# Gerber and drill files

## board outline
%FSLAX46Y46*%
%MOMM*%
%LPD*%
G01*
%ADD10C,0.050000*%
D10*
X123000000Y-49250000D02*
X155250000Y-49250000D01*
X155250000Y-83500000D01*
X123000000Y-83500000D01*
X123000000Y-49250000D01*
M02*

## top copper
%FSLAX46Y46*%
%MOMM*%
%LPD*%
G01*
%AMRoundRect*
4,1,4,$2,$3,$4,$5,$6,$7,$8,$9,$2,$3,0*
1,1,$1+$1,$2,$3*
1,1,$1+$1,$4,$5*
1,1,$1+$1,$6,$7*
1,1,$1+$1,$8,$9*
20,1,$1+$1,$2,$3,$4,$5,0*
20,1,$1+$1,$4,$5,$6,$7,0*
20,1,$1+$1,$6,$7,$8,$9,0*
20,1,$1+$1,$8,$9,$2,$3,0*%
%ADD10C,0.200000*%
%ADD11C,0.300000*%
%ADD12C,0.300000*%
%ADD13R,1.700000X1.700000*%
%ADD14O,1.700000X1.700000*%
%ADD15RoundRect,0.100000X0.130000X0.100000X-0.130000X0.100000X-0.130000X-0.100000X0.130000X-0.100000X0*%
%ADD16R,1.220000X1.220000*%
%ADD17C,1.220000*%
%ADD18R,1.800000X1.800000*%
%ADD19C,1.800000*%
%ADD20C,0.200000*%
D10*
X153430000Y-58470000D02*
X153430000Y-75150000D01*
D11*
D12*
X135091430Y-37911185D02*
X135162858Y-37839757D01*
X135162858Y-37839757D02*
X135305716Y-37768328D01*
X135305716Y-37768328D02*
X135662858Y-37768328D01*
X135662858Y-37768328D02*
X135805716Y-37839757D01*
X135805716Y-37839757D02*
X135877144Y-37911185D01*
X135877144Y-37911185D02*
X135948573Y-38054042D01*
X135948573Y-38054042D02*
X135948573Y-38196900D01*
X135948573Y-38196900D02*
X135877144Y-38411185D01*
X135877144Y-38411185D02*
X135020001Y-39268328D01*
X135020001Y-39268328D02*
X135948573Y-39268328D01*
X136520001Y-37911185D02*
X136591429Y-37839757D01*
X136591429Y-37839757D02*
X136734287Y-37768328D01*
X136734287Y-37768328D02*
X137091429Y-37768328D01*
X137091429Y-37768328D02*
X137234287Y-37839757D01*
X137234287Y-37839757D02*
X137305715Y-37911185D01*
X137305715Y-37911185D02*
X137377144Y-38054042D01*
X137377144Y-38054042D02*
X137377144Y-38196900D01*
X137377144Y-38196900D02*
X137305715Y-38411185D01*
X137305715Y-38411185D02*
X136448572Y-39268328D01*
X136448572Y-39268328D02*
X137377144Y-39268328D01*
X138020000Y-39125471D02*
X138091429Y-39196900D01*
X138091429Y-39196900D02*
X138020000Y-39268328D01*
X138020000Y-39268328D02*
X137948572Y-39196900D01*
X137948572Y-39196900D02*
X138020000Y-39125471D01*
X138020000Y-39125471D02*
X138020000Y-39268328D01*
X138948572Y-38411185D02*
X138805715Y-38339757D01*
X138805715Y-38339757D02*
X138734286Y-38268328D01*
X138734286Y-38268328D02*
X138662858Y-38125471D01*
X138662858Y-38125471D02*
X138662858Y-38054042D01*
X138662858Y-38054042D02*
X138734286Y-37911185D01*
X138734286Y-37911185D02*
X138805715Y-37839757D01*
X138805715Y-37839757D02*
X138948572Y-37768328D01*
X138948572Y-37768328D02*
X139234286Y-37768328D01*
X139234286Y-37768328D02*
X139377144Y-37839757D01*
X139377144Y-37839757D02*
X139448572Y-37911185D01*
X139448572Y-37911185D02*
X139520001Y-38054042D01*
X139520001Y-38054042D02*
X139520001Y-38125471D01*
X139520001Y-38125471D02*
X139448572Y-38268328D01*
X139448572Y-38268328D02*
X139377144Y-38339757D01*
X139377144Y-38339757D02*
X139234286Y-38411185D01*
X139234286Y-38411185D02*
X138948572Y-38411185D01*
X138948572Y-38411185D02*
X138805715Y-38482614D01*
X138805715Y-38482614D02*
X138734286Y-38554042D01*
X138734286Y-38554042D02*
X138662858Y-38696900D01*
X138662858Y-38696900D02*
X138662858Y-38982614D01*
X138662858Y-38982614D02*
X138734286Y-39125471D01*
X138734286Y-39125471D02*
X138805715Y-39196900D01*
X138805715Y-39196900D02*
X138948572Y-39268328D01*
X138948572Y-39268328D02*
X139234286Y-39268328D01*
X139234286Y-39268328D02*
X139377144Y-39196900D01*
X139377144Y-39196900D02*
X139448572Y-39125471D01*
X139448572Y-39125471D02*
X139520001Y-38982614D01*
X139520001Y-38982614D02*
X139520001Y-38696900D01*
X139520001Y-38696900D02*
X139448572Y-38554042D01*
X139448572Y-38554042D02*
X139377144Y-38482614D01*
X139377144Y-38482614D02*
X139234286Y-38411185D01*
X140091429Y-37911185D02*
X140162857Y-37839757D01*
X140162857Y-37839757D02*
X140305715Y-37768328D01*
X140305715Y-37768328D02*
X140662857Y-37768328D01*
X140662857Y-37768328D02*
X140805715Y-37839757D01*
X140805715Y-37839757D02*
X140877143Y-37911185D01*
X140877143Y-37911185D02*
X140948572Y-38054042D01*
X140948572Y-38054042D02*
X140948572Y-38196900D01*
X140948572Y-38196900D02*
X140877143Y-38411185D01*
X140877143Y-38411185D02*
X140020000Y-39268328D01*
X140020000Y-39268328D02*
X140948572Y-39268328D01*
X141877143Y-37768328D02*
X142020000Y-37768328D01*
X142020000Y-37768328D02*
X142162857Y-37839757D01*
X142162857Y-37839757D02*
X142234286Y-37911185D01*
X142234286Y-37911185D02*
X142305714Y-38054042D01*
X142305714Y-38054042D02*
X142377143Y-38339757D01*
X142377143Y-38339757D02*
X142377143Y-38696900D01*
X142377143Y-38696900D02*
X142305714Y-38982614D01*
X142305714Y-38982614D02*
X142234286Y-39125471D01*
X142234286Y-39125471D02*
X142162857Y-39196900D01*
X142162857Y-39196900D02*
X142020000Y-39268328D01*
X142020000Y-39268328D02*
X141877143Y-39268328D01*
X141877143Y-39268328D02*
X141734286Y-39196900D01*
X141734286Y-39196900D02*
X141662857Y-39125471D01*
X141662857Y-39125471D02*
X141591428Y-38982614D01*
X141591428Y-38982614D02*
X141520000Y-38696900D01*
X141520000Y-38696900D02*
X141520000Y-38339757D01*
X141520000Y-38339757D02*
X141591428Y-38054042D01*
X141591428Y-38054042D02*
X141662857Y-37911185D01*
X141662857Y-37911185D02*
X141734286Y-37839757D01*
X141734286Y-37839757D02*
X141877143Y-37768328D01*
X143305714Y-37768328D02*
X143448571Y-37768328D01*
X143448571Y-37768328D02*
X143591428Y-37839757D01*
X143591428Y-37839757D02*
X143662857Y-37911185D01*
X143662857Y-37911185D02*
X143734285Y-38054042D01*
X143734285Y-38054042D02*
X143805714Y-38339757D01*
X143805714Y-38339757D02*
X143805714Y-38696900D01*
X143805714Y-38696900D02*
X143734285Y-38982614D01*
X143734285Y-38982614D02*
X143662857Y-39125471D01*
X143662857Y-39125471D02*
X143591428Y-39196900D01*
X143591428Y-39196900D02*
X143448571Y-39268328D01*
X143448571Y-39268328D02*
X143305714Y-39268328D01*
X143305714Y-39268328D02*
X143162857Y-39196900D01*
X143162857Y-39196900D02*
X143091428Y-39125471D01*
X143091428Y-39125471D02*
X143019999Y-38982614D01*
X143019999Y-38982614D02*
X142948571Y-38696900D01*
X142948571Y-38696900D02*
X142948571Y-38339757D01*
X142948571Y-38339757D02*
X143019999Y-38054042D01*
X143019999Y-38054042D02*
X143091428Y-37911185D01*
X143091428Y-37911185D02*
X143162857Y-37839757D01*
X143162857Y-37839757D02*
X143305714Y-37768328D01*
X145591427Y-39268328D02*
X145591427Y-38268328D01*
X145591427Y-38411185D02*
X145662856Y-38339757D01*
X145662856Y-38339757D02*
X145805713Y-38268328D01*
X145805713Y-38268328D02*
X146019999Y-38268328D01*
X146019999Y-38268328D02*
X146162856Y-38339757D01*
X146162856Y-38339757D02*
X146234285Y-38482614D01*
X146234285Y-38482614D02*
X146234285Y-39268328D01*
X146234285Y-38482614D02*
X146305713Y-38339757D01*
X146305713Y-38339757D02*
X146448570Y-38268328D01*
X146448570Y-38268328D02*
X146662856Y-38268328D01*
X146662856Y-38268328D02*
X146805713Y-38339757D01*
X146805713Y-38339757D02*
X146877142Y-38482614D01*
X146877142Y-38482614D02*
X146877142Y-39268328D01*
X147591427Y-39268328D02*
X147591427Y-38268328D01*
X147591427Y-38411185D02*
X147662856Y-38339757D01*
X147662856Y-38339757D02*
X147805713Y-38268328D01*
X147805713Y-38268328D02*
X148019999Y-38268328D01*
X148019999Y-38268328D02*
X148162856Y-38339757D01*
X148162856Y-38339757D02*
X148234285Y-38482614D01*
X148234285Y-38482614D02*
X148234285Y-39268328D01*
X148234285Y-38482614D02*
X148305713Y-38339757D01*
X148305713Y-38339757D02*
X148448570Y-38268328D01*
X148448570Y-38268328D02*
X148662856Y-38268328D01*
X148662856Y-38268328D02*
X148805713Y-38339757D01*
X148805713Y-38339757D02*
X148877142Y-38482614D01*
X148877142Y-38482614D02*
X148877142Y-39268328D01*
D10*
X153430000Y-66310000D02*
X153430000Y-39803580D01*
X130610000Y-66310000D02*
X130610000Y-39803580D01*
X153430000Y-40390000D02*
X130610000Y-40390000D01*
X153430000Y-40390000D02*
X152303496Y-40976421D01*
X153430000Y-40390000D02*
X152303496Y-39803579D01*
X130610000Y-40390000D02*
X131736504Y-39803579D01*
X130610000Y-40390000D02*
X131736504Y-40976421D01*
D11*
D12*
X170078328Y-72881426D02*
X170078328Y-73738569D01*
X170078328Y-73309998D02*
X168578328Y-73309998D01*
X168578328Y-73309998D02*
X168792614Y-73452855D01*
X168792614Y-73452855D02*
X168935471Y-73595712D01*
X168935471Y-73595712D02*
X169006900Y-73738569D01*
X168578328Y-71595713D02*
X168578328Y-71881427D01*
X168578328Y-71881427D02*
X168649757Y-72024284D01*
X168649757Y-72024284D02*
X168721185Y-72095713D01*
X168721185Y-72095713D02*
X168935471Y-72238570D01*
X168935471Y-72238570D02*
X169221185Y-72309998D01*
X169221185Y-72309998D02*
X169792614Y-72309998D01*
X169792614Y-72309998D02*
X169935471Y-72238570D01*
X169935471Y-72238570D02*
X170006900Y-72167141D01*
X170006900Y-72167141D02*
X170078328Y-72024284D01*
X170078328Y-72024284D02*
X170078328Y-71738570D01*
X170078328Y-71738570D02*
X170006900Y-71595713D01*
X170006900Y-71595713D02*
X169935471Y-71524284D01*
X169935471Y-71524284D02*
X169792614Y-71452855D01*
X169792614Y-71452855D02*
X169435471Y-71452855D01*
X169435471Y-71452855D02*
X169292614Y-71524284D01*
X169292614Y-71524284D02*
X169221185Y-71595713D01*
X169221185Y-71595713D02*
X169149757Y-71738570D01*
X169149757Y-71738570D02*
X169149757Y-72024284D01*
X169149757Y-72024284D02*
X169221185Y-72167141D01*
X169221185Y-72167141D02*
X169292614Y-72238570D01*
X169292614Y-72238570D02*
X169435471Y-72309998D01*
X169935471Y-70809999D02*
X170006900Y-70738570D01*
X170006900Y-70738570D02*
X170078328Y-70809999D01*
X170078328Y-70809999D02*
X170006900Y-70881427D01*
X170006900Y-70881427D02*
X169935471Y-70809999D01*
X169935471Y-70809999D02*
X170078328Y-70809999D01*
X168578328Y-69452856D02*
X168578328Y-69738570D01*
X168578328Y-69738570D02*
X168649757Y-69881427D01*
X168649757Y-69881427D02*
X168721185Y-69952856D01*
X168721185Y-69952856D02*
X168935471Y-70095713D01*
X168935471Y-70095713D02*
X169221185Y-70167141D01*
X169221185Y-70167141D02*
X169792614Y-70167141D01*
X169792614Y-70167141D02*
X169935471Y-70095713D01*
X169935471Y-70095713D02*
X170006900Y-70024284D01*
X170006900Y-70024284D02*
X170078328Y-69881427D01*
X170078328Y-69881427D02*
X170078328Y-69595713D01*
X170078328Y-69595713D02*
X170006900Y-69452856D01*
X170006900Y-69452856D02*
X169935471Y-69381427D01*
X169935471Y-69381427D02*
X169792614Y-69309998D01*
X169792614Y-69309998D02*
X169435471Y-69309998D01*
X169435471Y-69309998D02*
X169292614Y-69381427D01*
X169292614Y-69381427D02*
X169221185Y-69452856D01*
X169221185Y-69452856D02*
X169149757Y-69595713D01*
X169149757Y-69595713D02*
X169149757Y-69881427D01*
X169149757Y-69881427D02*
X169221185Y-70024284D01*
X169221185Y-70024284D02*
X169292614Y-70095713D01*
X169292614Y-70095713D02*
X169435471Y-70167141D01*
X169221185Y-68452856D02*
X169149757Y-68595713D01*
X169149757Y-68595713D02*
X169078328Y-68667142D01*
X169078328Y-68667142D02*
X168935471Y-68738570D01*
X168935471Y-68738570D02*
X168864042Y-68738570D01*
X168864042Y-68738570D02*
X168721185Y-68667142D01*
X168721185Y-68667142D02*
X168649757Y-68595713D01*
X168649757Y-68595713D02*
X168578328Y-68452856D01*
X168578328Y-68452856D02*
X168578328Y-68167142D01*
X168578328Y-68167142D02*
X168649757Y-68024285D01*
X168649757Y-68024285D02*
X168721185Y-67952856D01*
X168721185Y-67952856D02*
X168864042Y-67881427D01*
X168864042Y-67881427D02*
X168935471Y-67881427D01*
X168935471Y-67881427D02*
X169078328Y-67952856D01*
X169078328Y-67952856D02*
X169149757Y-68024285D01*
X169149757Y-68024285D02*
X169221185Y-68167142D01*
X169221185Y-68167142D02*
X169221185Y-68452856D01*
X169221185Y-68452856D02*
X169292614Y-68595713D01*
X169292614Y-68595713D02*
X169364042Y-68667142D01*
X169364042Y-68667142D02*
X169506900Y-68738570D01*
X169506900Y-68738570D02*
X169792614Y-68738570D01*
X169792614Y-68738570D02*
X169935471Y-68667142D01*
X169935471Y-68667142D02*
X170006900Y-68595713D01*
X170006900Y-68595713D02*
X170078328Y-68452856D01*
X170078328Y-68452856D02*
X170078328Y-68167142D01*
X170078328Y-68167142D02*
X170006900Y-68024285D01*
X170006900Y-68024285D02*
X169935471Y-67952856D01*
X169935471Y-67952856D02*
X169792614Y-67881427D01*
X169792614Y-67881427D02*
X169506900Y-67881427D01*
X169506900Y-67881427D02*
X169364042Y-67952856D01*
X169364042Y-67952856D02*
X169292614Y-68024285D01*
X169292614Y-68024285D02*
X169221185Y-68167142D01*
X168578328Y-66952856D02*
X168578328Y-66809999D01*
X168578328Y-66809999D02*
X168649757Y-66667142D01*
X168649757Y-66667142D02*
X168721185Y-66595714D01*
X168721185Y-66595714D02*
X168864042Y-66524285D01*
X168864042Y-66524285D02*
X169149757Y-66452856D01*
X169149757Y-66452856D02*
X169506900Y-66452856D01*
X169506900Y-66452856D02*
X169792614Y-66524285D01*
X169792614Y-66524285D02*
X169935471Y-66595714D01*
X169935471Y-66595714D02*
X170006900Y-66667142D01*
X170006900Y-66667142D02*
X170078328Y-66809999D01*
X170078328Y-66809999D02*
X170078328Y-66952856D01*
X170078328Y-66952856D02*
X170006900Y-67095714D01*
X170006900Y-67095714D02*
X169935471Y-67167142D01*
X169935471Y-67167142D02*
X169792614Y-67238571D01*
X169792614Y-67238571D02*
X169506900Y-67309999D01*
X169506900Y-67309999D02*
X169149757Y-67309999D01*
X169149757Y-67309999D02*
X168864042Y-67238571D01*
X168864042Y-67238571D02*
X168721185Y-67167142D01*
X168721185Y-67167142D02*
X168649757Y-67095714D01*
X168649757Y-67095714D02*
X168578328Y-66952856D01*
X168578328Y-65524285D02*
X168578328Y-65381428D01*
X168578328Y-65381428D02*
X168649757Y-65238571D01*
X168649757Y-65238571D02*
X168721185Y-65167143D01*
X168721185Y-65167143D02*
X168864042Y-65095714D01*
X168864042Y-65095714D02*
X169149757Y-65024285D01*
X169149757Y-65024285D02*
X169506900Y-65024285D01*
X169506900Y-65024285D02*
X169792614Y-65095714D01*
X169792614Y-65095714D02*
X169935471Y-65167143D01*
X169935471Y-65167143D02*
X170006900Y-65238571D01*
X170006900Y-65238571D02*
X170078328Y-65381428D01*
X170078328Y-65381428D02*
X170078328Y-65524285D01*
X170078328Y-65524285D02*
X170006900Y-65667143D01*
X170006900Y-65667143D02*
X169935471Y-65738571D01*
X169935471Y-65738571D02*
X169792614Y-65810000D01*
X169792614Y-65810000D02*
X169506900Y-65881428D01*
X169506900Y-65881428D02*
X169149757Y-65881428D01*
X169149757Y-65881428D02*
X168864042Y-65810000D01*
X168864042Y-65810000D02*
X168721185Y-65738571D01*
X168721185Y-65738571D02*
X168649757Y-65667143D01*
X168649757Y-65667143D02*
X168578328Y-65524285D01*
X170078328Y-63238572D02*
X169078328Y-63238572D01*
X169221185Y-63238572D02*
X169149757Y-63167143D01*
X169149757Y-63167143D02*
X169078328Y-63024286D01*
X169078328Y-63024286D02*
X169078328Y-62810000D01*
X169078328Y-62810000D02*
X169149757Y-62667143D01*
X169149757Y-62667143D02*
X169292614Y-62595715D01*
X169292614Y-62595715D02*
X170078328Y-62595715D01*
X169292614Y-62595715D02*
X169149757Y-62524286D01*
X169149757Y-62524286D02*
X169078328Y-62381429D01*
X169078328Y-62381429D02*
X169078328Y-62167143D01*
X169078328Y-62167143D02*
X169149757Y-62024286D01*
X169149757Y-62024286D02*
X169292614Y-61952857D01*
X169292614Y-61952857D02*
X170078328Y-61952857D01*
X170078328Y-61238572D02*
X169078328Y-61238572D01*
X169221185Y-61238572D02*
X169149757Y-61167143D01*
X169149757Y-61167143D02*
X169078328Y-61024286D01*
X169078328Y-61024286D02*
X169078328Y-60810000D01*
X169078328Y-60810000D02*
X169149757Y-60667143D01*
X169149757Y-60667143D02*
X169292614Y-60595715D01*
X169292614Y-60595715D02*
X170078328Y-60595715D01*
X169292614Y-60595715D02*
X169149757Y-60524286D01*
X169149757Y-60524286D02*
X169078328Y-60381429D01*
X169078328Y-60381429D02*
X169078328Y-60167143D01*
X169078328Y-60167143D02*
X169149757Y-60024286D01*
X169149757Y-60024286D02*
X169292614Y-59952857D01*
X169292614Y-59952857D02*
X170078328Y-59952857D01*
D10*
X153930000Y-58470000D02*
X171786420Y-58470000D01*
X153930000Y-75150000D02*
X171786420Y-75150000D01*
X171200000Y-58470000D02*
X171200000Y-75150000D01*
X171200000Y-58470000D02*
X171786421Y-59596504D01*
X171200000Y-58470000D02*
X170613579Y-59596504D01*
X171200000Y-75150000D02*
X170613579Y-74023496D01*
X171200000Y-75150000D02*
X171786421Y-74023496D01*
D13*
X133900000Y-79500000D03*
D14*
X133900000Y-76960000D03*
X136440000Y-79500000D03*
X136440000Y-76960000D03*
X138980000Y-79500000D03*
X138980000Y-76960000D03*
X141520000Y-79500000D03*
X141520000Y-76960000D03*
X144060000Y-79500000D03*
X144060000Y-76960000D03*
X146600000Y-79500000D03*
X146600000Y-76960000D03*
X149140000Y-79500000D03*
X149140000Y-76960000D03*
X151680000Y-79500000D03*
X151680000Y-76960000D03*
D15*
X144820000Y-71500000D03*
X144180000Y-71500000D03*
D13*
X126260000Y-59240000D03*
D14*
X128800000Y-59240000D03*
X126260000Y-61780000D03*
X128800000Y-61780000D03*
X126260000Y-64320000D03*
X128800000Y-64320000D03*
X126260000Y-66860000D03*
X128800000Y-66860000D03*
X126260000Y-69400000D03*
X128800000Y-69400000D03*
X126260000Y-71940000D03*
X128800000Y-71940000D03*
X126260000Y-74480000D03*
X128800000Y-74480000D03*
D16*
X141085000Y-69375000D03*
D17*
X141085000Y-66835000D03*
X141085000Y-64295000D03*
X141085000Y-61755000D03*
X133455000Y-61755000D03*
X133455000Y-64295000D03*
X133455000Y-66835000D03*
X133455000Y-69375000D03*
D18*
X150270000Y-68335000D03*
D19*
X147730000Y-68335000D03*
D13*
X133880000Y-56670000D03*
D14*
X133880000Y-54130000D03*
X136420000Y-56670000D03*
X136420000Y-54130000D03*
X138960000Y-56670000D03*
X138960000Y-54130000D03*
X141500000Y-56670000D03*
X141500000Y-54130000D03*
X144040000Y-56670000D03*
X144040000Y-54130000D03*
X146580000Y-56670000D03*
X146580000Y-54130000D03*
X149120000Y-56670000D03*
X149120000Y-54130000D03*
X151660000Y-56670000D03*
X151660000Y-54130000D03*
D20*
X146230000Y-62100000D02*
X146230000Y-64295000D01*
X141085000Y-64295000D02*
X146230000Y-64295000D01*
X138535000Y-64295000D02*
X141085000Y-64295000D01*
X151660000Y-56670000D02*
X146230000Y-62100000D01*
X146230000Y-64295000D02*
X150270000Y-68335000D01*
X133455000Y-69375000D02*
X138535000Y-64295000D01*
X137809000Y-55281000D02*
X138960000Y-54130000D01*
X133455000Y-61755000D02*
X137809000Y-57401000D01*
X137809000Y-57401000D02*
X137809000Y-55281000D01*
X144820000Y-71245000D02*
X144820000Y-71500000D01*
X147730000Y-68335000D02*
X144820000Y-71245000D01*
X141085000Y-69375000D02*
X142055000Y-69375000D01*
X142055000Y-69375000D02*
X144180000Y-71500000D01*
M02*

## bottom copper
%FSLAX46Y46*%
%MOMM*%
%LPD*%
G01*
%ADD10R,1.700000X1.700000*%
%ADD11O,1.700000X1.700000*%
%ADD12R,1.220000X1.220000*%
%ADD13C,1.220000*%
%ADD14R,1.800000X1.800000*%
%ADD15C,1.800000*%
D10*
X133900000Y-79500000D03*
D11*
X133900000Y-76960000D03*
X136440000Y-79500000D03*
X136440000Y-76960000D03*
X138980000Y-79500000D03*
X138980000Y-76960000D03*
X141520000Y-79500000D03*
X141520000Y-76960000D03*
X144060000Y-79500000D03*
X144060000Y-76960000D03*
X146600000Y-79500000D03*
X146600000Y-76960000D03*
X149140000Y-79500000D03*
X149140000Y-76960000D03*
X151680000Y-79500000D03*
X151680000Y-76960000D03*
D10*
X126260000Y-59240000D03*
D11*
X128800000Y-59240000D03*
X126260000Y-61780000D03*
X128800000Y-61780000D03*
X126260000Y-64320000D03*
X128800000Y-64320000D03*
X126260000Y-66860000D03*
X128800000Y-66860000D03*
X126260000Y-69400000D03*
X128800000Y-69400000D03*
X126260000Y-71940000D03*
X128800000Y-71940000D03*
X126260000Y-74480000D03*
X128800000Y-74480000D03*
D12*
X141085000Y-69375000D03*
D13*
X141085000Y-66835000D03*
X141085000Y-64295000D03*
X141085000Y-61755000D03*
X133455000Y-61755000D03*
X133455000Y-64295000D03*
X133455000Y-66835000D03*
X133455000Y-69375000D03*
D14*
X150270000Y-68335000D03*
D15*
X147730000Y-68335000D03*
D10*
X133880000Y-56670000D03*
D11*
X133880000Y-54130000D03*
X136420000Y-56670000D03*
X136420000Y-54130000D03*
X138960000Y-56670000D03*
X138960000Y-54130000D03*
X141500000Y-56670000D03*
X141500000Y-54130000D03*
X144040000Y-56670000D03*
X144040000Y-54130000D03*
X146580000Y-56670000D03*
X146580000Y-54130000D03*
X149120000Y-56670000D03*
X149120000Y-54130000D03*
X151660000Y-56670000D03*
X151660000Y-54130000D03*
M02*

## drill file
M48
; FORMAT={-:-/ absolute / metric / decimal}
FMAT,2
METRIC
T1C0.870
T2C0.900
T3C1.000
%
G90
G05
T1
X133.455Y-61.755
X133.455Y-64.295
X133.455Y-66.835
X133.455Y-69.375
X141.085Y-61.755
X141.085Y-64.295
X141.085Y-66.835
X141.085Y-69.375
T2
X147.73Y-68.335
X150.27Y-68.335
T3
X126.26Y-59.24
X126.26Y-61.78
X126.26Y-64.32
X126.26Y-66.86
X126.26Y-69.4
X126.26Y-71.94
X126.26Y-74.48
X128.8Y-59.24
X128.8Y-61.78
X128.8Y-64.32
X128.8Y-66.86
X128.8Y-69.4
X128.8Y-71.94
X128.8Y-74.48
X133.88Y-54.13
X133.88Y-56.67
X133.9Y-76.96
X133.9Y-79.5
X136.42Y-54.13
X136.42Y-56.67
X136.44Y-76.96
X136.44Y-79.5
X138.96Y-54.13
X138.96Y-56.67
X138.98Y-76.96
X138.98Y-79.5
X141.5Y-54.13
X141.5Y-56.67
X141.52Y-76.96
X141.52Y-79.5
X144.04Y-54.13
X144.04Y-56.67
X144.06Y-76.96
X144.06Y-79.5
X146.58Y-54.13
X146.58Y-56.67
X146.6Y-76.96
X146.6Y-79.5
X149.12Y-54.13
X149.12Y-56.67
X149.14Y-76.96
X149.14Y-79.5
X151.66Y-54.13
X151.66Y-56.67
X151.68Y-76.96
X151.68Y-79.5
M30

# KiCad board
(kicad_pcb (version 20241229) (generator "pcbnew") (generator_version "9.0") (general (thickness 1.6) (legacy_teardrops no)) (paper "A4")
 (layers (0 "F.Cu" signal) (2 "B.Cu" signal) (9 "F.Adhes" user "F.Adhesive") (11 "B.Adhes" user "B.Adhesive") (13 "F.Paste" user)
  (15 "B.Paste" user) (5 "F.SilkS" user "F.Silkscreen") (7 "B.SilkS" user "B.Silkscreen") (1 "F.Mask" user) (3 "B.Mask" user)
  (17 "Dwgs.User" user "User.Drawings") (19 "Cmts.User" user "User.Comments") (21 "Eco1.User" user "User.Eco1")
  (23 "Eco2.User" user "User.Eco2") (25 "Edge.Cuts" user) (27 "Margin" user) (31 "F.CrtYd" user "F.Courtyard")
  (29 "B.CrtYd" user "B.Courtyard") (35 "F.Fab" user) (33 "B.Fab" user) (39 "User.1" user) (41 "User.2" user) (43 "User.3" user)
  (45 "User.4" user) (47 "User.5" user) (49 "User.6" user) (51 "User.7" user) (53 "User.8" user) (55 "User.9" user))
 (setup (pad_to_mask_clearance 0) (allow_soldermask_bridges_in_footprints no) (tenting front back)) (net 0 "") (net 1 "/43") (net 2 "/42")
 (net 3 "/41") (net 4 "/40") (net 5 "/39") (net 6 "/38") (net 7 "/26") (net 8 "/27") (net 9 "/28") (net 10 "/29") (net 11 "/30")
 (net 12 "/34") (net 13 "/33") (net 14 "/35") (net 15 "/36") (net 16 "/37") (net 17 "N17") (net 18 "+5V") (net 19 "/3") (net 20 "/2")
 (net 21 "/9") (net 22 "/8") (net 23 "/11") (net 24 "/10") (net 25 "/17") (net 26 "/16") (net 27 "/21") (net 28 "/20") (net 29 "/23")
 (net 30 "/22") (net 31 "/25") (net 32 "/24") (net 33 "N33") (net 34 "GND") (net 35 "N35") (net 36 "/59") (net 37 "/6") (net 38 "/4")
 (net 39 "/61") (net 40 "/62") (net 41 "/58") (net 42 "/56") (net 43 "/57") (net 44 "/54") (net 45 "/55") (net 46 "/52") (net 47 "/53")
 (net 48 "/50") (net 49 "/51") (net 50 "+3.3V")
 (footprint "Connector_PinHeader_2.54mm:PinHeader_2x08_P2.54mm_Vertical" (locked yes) (layer "F.Cu") (at 133.9 79.5 90)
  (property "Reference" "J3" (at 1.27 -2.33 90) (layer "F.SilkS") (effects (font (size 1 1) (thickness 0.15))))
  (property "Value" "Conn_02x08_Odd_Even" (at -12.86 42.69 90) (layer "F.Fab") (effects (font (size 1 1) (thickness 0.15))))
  (pad "1" thru_hole rect (at 0 0 90) (size 1.7 1.7) (drill 1) (layers "*.Cu" "*.Mask") (remove_unused_layers no) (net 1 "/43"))
  (pad "2" thru_hole oval (at 2.54 0 90) (size 1.7 1.7) (drill 1) (layers "*.Cu" "*.Mask") (remove_unused_layers no) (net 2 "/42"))
  (pad "3" thru_hole oval (at 0 2.54 90) (size 1.7 1.7) (drill 1) (layers "*.Cu" "*.Mask") (remove_unused_layers no) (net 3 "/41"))
  (pad "4" thru_hole oval (at 2.54 2.54 90) (size 1.7 1.7) (drill 1) (layers "*.Cu" "*.Mask") (remove_unused_layers no) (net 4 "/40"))
  (pad "5" thru_hole oval (at 0 5.08 90) (size 1.7 1.7) (drill 1) (layers "*.Cu" "*.Mask") (remove_unused_layers no) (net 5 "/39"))
  (pad "6" thru_hole oval (at 2.54 5.08 90) (size 1.7 1.7) (drill 1) (layers "*.Cu" "*.Mask") (remove_unused_layers no) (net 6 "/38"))
  (pad "7" thru_hole oval (at 0 7.62 90) (size 1.7 1.7) (drill 1) (layers "*.Cu" "*.Mask") (remove_unused_layers no) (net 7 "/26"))
  (pad "8" thru_hole oval (at 2.54 7.62 90) (size 1.7 1.7) (drill 1) (layers "*.Cu" "*.Mask") (remove_unused_layers no) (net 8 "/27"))
  (pad "9" thru_hole oval (at 0 10.16 90) (size 1.7 1.7) (drill 1) (layers "*.Cu" "*.Mask") (remove_unused_layers no) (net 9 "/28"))
  (pad "10" thru_hole oval (at 2.54 10.16 90) (size 1.7 1.7) (drill 1) (layers "*.Cu" "*.Mask") (remove_unused_layers no) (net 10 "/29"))
  (pad "11" thru_hole oval (at 0 12.7 90) (size 1.7 1.7) (drill 1) (layers "*.Cu" "*.Mask") (remove_unused_layers no) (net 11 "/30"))
  (pad "12" thru_hole oval (at 2.54 12.7 90) (size 1.7 1.7) (drill 1) (layers "*.Cu" "*.Mask") (remove_unused_layers no) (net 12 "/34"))
  (pad "13" thru_hole oval (at 0 15.24 90) (size 1.7 1.7) (drill 1) (layers "*.Cu" "*.Mask") (remove_unused_layers no) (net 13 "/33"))
  (pad "14" thru_hole oval (at 2.54 15.24 90) (size 1.7 1.7) (drill 1) (layers "*.Cu" "*.Mask") (remove_unused_layers no) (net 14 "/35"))
  (pad "15" thru_hole oval (at 0 17.78 90) (size 1.7 1.7) (drill 1) (layers "*.Cu" "*.Mask") (remove_unused_layers no) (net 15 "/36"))
  (pad "16" thru_hole oval (at 2.54 17.78 90) (size 1.7 1.7) (drill 1) (layers "*.Cu" "*.Mask") (remove_unused_layers no) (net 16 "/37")))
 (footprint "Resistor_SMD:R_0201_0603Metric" (layer "F.Cu") (at 144.5 71.5 180)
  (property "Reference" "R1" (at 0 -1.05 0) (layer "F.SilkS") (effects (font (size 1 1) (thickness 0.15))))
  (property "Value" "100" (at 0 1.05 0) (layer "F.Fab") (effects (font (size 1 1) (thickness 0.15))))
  (pad "" smd roundrect (at -0.345 0 180) (size 0.318 0.36) (layers "F.Paste") (roundrect_rratio 0.25))
  (pad "" smd roundrect (at 0.345 0 180) (size 0.318 0.36) (layers "F.Paste") (roundrect_rratio 0.25))
  (pad "1" smd roundrect (at -0.32 0 180) (size 0.46 0.4) (layers "F.Cu" "F.Mask") (roundrect_rratio 0.25) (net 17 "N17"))
  (pad "2" smd roundrect (at 0.32 0 180) (size 0.46 0.4) (layers "F.Cu" "F.Mask") (roundrect_rratio 0.25) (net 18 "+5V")))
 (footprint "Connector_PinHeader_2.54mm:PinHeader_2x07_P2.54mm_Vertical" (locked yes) (layer "F.Cu") (at 126.26 59.24)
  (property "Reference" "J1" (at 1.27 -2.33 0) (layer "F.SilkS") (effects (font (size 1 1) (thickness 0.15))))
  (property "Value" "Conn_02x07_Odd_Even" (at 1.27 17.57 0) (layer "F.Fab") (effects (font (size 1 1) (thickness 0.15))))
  (pad "1" thru_hole rect (at 0 0) (size 1.7 1.7) (drill 1) (layers "*.Cu" "*.Mask") (remove_unused_layers no) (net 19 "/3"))
  (pad "2" thru_hole oval (at 2.54 0) (size 1.7 1.7) (drill 1) (layers "*.Cu" "*.Mask") (remove_unused_layers no) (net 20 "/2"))
  (pad "3" thru_hole oval (at 0 2.54) (size 1.7 1.7) (drill 1) (layers "*.Cu" "*.Mask") (remove_unused_layers no) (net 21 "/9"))
  (pad "4" thru_hole oval (at 2.54 2.54) (size 1.7 1.7) (drill 1) (layers "*.Cu" "*.Mask") (remove_unused_layers no) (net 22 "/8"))
  (pad "5" thru_hole oval (at 0 5.08) (size 1.7 1.7) (drill 1) (layers "*.Cu" "*.Mask") (remove_unused_layers no) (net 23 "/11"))
  (pad "6" thru_hole oval (at 2.54 5.08) (size 1.7 1.7) (drill 1) (layers "*.Cu" "*.Mask") (remove_unused_layers no) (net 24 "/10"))
  (pad "7" thru_hole oval (at 0 7.62) (size 1.7 1.7) (drill 1) (layers "*.Cu" "*.Mask") (remove_unused_layers no) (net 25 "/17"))
  (pad "8" thru_hole oval (at 2.54 7.62) (size 1.7 1.7) (drill 1) (layers "*.Cu" "*.Mask") (remove_unused_layers no) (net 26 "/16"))
  (pad "9" thru_hole oval (at 0 10.16) (size 1.7 1.7) (drill 1) (layers "*.Cu" "*.Mask") (remove_unused_layers no) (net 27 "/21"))
  (pad "10" thru_hole oval (at 2.54 10.16) (size 1.7 1.7) (drill 1) (layers "*.Cu" "*.Mask") (remove_unused_layers no) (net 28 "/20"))
  (pad "11" thru_hole oval (at 0 12.7) (size 1.7 1.7) (drill 1) (layers "*.Cu" "*.Mask") (remove_unused_layers no) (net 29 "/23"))
  (pad "12" thru_hole oval (at 2.54 12.7) (size 1.7 1.7) (drill 1) (layers "*.Cu" "*.Mask") (remove_unused_layers no) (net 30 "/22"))
  (pad "13" thru_hole oval (at 0 15.24) (size 1.7 1.7) (drill 1) (layers "*.Cu" "*.Mask") (remove_unused_layers no) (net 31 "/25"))
  (pad "14" thru_hole oval (at 2.54 15.24) (size 1.7 1.7) (drill 1) (layers "*.Cu" "*.Mask") (remove_unused_layers no) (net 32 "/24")))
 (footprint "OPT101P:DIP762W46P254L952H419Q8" (layer "F.Cu") (at 137.27 65.565 180)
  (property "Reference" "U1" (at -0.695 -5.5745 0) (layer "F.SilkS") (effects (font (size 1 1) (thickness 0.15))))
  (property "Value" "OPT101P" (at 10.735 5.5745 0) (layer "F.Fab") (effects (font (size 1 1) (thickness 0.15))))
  (pad "1" thru_hole rect (at -3.815 -3.81 180) (size 1.22 1.22) (drill 0.87) (layers "*.Cu" "*.Mask") (remove_unused_layers no)
   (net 18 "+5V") (solder_mask_margin 0.102))
  (pad "2" thru_hole circle (at -3.815 -1.27 180) (size 1.22 1.22) (drill 0.87) (layers "*.Cu" "*.Mask") (remove_unused_layers no)
   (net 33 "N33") (solder_mask_margin 0.102))
  (pad "3" thru_hole circle (at -3.815 1.27 180) (size 1.22 1.22) (drill 0.87) (layers "*.Cu" "*.Mask") (remove_unused_layers no)
   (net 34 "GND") (solder_mask_margin 0.102))
  (pad "4" thru_hole circle (at -3.815 3.81 180) (size 1.22 1.22) (drill 0.87) (layers "*.Cu" "*.Mask") (remove_unused_layers no)
   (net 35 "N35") (solder_mask_margin 0.102))
  (pad "5" thru_hole circle (at 3.815 3.81 180) (size 1.22 1.22) (drill 0.87) (layers "*.Cu" "*.Mask") (remove_unused_layers no)
   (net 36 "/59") (solder_mask_margin 0.102))
  (pad "6" thru_hole circle (at 3.815 1.27 180) (size 1.22 1.22) (drill 0.87) (layers "*.Cu" "*.Mask") (remove_unused_layers no)
   (solder_mask_margin 0.102))
  (pad "7" thru_hole circle (at 3.815 -1.27 180) (size 1.22 1.22) (drill 0.87) (layers "*.Cu" "*.Mask") (remove_unused_layers no)
   (solder_mask_margin 0.102))
  (pad "8" thru_hole circle (at 3.815 -3.81 180) (size 1.22 1.22) (drill 0.87) (layers "*.Cu" "*.Mask") (remove_unused_layers no)
   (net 34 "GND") (solder_mask_margin 0.102)))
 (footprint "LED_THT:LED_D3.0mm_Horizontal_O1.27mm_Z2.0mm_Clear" (layer "F.Cu") (at 150.27 68.335 180)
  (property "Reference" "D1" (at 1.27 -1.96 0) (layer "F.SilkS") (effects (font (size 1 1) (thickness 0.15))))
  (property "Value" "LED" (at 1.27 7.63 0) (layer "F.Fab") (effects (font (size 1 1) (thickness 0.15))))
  (pad "1" thru_hole rect (at 0 0 180) (size 1.8 1.8) (drill 0.9) (layers "*.Cu" "*.Mask") (remove_unused_layers no) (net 34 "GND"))
  (pad "2" thru_hole circle (at 2.54 0 180) (size 1.8 1.8) (drill 0.9) (layers "*.Cu" "*.Mask") (remove_unused_layers no) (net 17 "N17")))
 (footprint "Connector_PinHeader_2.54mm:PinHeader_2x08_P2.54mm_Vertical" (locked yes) (layer "F.Cu") (at 133.88 56.67 90)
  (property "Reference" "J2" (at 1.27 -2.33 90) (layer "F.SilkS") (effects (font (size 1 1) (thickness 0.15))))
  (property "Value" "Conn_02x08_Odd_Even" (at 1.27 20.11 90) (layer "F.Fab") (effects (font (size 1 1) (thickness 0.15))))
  (pad "1" thru_hole rect (at 0 0 90) (size 1.7 1.7) (drill 1) (layers "*.Cu" "*.Mask") (remove_unused_layers no) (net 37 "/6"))
  (pad "2" thru_hole oval (at 2.54 0 90) (size 1.7 1.7) (drill 1) (layers "*.Cu" "*.Mask") (remove_unused_layers no) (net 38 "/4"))
  (pad "3" thru_hole oval (at 0 2.54 90) (size 1.7 1.7) (drill 1) (layers "*.Cu" "*.Mask") (remove_unused_layers no) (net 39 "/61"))
  (pad "4" thru_hole oval (at 2.54 2.54 90) (size 1.7 1.7) (drill 1) (layers "*.Cu" "*.Mask") (remove_unused_layers no) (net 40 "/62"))
  (pad "5" thru_hole oval (at 0 5.08 90) (size 1.7 1.7) (drill 1) (layers "*.Cu" "*.Mask") (remove_unused_layers no) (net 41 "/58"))
  (pad "6" thru_hole oval (at 2.54 5.08 90) (size 1.7 1.7) (drill 1) (layers "*.Cu" "*.Mask") (remove_unused_layers no) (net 36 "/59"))
  (pad "7" thru_hole oval (at 0 7.62 90) (size 1.7 1.7) (drill 1) (layers "*.Cu" "*.Mask") (remove_unused_layers no) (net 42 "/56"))
  (pad "8" thru_hole oval (at 2.54 7.62 90) (size 1.7 1.7) (drill 1) (layers "*.Cu" "*.Mask") (remove_unused_layers no) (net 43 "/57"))
  (pad "9" thru_hole oval (at 0 10.16 90) (size 1.7 1.7) (drill 1) (layers "*.Cu" "*.Mask") (remove_unused_layers no) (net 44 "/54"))
  (pad "10" thru_hole oval (at 2.54 10.16 90) (size 1.7 1.7) (drill 1) (layers "*.Cu" "*.Mask") (remove_unused_layers no) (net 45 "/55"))
  (pad "11" thru_hole oval (at 0 12.7 90) (size 1.7 1.7) (drill 1) (layers "*.Cu" "*.Mask") (remove_unused_layers no) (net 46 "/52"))
  (pad "12" thru_hole oval (at 2.54 12.7 90) (size 1.7 1.7) (drill 1) (layers "*.Cu" "*.Mask") (remove_unused_layers no) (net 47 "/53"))
  (pad "13" thru_hole oval (at 0 15.24 90) (size 1.7 1.7) (drill 1) (layers "*.Cu" "*.Mask") (remove_unused_layers no) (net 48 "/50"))
  (pad "14" thru_hole oval (at 2.54 15.24 90) (size 1.7 1.7) (drill 1) (layers "*.Cu" "*.Mask") (remove_unused_layers no) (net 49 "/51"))
  (pad "15" thru_hole oval (at 0 17.78 90) (size 1.7 1.7) (drill 1) (layers "*.Cu" "*.Mask") (remove_unused_layers no) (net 34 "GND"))
  (pad "16" thru_hole oval (at 2.54 17.78 90) (size 1.7 1.7) (drill 1) (layers "*.Cu" "*.Mask") (remove_unused_layers no) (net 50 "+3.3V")))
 (gr_line (start 153.43 58.47) (end 153.43 75.15) (stroke (width 0.2) (type default)) (layer "F.Cu"))
 (gr_rect (start 123 49.25) (end 155.25 83.5) (stroke (width 0.05) (type default)) (fill no) (layer "Edge.Cuts"))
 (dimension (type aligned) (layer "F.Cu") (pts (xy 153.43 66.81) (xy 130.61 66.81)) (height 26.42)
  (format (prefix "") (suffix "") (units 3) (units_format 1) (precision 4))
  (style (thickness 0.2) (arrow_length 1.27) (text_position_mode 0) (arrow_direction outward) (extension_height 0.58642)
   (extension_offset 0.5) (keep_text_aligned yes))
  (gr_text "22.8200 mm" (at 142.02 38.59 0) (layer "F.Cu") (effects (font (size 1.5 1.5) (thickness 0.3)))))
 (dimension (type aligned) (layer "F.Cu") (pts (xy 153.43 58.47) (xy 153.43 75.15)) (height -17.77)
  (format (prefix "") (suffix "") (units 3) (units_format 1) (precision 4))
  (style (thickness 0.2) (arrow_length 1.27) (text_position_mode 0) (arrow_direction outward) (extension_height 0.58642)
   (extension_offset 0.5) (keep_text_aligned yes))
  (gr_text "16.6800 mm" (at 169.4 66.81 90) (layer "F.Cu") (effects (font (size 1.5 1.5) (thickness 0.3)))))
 (segment (start 146.23 62.1) (end 146.23 64.295) (width 0.2) (layer "F.Cu") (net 34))
 (segment (start 141.085 64.295) (end 146.23 64.295) (width 0.2) (layer "F.Cu") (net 34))
 (segment (start 138.535 64.295) (end 141.085 64.295) (width 0.2) (layer "F.Cu") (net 34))
 (segment (start 151.66 56.67) (end 146.23 62.1) (width 0.2) (layer "F.Cu") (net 34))
 (segment (start 146.23 64.295) (end 150.27 68.335) (width 0.2) (layer "F.Cu") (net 34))
 (segment (start 133.455 69.375) (end 138.535 64.295) (width 0.2) (layer "F.Cu") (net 34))
 (segment (start 137.809 55.281) (end 138.96 54.13) (width 0.2) (layer "F.Cu") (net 36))
 (segment (start 133.455 61.755) (end 137.809 57.401) (width 0.2) (layer "F.Cu") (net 36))
 (segment (start 137.809 57.401) (end 137.809 55.281) (width 0.2) (layer "F.Cu") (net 36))
 (segment (start 144.82 71.245) (end 144.82 71.5) (width 0.2) (layer "F.Cu") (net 17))
 (segment (start 147.73 68.335) (end 144.82 71.245) (width 0.2) (layer "F.Cu") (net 17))
 (segment (start 141.085 69.375) (end 142.055 69.375) (width 0.2) (layer "F.Cu") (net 18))
 (segment (start 142.055 69.375) (end 144.18 71.5) (width 0.2) (layer "F.Cu") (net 18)))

